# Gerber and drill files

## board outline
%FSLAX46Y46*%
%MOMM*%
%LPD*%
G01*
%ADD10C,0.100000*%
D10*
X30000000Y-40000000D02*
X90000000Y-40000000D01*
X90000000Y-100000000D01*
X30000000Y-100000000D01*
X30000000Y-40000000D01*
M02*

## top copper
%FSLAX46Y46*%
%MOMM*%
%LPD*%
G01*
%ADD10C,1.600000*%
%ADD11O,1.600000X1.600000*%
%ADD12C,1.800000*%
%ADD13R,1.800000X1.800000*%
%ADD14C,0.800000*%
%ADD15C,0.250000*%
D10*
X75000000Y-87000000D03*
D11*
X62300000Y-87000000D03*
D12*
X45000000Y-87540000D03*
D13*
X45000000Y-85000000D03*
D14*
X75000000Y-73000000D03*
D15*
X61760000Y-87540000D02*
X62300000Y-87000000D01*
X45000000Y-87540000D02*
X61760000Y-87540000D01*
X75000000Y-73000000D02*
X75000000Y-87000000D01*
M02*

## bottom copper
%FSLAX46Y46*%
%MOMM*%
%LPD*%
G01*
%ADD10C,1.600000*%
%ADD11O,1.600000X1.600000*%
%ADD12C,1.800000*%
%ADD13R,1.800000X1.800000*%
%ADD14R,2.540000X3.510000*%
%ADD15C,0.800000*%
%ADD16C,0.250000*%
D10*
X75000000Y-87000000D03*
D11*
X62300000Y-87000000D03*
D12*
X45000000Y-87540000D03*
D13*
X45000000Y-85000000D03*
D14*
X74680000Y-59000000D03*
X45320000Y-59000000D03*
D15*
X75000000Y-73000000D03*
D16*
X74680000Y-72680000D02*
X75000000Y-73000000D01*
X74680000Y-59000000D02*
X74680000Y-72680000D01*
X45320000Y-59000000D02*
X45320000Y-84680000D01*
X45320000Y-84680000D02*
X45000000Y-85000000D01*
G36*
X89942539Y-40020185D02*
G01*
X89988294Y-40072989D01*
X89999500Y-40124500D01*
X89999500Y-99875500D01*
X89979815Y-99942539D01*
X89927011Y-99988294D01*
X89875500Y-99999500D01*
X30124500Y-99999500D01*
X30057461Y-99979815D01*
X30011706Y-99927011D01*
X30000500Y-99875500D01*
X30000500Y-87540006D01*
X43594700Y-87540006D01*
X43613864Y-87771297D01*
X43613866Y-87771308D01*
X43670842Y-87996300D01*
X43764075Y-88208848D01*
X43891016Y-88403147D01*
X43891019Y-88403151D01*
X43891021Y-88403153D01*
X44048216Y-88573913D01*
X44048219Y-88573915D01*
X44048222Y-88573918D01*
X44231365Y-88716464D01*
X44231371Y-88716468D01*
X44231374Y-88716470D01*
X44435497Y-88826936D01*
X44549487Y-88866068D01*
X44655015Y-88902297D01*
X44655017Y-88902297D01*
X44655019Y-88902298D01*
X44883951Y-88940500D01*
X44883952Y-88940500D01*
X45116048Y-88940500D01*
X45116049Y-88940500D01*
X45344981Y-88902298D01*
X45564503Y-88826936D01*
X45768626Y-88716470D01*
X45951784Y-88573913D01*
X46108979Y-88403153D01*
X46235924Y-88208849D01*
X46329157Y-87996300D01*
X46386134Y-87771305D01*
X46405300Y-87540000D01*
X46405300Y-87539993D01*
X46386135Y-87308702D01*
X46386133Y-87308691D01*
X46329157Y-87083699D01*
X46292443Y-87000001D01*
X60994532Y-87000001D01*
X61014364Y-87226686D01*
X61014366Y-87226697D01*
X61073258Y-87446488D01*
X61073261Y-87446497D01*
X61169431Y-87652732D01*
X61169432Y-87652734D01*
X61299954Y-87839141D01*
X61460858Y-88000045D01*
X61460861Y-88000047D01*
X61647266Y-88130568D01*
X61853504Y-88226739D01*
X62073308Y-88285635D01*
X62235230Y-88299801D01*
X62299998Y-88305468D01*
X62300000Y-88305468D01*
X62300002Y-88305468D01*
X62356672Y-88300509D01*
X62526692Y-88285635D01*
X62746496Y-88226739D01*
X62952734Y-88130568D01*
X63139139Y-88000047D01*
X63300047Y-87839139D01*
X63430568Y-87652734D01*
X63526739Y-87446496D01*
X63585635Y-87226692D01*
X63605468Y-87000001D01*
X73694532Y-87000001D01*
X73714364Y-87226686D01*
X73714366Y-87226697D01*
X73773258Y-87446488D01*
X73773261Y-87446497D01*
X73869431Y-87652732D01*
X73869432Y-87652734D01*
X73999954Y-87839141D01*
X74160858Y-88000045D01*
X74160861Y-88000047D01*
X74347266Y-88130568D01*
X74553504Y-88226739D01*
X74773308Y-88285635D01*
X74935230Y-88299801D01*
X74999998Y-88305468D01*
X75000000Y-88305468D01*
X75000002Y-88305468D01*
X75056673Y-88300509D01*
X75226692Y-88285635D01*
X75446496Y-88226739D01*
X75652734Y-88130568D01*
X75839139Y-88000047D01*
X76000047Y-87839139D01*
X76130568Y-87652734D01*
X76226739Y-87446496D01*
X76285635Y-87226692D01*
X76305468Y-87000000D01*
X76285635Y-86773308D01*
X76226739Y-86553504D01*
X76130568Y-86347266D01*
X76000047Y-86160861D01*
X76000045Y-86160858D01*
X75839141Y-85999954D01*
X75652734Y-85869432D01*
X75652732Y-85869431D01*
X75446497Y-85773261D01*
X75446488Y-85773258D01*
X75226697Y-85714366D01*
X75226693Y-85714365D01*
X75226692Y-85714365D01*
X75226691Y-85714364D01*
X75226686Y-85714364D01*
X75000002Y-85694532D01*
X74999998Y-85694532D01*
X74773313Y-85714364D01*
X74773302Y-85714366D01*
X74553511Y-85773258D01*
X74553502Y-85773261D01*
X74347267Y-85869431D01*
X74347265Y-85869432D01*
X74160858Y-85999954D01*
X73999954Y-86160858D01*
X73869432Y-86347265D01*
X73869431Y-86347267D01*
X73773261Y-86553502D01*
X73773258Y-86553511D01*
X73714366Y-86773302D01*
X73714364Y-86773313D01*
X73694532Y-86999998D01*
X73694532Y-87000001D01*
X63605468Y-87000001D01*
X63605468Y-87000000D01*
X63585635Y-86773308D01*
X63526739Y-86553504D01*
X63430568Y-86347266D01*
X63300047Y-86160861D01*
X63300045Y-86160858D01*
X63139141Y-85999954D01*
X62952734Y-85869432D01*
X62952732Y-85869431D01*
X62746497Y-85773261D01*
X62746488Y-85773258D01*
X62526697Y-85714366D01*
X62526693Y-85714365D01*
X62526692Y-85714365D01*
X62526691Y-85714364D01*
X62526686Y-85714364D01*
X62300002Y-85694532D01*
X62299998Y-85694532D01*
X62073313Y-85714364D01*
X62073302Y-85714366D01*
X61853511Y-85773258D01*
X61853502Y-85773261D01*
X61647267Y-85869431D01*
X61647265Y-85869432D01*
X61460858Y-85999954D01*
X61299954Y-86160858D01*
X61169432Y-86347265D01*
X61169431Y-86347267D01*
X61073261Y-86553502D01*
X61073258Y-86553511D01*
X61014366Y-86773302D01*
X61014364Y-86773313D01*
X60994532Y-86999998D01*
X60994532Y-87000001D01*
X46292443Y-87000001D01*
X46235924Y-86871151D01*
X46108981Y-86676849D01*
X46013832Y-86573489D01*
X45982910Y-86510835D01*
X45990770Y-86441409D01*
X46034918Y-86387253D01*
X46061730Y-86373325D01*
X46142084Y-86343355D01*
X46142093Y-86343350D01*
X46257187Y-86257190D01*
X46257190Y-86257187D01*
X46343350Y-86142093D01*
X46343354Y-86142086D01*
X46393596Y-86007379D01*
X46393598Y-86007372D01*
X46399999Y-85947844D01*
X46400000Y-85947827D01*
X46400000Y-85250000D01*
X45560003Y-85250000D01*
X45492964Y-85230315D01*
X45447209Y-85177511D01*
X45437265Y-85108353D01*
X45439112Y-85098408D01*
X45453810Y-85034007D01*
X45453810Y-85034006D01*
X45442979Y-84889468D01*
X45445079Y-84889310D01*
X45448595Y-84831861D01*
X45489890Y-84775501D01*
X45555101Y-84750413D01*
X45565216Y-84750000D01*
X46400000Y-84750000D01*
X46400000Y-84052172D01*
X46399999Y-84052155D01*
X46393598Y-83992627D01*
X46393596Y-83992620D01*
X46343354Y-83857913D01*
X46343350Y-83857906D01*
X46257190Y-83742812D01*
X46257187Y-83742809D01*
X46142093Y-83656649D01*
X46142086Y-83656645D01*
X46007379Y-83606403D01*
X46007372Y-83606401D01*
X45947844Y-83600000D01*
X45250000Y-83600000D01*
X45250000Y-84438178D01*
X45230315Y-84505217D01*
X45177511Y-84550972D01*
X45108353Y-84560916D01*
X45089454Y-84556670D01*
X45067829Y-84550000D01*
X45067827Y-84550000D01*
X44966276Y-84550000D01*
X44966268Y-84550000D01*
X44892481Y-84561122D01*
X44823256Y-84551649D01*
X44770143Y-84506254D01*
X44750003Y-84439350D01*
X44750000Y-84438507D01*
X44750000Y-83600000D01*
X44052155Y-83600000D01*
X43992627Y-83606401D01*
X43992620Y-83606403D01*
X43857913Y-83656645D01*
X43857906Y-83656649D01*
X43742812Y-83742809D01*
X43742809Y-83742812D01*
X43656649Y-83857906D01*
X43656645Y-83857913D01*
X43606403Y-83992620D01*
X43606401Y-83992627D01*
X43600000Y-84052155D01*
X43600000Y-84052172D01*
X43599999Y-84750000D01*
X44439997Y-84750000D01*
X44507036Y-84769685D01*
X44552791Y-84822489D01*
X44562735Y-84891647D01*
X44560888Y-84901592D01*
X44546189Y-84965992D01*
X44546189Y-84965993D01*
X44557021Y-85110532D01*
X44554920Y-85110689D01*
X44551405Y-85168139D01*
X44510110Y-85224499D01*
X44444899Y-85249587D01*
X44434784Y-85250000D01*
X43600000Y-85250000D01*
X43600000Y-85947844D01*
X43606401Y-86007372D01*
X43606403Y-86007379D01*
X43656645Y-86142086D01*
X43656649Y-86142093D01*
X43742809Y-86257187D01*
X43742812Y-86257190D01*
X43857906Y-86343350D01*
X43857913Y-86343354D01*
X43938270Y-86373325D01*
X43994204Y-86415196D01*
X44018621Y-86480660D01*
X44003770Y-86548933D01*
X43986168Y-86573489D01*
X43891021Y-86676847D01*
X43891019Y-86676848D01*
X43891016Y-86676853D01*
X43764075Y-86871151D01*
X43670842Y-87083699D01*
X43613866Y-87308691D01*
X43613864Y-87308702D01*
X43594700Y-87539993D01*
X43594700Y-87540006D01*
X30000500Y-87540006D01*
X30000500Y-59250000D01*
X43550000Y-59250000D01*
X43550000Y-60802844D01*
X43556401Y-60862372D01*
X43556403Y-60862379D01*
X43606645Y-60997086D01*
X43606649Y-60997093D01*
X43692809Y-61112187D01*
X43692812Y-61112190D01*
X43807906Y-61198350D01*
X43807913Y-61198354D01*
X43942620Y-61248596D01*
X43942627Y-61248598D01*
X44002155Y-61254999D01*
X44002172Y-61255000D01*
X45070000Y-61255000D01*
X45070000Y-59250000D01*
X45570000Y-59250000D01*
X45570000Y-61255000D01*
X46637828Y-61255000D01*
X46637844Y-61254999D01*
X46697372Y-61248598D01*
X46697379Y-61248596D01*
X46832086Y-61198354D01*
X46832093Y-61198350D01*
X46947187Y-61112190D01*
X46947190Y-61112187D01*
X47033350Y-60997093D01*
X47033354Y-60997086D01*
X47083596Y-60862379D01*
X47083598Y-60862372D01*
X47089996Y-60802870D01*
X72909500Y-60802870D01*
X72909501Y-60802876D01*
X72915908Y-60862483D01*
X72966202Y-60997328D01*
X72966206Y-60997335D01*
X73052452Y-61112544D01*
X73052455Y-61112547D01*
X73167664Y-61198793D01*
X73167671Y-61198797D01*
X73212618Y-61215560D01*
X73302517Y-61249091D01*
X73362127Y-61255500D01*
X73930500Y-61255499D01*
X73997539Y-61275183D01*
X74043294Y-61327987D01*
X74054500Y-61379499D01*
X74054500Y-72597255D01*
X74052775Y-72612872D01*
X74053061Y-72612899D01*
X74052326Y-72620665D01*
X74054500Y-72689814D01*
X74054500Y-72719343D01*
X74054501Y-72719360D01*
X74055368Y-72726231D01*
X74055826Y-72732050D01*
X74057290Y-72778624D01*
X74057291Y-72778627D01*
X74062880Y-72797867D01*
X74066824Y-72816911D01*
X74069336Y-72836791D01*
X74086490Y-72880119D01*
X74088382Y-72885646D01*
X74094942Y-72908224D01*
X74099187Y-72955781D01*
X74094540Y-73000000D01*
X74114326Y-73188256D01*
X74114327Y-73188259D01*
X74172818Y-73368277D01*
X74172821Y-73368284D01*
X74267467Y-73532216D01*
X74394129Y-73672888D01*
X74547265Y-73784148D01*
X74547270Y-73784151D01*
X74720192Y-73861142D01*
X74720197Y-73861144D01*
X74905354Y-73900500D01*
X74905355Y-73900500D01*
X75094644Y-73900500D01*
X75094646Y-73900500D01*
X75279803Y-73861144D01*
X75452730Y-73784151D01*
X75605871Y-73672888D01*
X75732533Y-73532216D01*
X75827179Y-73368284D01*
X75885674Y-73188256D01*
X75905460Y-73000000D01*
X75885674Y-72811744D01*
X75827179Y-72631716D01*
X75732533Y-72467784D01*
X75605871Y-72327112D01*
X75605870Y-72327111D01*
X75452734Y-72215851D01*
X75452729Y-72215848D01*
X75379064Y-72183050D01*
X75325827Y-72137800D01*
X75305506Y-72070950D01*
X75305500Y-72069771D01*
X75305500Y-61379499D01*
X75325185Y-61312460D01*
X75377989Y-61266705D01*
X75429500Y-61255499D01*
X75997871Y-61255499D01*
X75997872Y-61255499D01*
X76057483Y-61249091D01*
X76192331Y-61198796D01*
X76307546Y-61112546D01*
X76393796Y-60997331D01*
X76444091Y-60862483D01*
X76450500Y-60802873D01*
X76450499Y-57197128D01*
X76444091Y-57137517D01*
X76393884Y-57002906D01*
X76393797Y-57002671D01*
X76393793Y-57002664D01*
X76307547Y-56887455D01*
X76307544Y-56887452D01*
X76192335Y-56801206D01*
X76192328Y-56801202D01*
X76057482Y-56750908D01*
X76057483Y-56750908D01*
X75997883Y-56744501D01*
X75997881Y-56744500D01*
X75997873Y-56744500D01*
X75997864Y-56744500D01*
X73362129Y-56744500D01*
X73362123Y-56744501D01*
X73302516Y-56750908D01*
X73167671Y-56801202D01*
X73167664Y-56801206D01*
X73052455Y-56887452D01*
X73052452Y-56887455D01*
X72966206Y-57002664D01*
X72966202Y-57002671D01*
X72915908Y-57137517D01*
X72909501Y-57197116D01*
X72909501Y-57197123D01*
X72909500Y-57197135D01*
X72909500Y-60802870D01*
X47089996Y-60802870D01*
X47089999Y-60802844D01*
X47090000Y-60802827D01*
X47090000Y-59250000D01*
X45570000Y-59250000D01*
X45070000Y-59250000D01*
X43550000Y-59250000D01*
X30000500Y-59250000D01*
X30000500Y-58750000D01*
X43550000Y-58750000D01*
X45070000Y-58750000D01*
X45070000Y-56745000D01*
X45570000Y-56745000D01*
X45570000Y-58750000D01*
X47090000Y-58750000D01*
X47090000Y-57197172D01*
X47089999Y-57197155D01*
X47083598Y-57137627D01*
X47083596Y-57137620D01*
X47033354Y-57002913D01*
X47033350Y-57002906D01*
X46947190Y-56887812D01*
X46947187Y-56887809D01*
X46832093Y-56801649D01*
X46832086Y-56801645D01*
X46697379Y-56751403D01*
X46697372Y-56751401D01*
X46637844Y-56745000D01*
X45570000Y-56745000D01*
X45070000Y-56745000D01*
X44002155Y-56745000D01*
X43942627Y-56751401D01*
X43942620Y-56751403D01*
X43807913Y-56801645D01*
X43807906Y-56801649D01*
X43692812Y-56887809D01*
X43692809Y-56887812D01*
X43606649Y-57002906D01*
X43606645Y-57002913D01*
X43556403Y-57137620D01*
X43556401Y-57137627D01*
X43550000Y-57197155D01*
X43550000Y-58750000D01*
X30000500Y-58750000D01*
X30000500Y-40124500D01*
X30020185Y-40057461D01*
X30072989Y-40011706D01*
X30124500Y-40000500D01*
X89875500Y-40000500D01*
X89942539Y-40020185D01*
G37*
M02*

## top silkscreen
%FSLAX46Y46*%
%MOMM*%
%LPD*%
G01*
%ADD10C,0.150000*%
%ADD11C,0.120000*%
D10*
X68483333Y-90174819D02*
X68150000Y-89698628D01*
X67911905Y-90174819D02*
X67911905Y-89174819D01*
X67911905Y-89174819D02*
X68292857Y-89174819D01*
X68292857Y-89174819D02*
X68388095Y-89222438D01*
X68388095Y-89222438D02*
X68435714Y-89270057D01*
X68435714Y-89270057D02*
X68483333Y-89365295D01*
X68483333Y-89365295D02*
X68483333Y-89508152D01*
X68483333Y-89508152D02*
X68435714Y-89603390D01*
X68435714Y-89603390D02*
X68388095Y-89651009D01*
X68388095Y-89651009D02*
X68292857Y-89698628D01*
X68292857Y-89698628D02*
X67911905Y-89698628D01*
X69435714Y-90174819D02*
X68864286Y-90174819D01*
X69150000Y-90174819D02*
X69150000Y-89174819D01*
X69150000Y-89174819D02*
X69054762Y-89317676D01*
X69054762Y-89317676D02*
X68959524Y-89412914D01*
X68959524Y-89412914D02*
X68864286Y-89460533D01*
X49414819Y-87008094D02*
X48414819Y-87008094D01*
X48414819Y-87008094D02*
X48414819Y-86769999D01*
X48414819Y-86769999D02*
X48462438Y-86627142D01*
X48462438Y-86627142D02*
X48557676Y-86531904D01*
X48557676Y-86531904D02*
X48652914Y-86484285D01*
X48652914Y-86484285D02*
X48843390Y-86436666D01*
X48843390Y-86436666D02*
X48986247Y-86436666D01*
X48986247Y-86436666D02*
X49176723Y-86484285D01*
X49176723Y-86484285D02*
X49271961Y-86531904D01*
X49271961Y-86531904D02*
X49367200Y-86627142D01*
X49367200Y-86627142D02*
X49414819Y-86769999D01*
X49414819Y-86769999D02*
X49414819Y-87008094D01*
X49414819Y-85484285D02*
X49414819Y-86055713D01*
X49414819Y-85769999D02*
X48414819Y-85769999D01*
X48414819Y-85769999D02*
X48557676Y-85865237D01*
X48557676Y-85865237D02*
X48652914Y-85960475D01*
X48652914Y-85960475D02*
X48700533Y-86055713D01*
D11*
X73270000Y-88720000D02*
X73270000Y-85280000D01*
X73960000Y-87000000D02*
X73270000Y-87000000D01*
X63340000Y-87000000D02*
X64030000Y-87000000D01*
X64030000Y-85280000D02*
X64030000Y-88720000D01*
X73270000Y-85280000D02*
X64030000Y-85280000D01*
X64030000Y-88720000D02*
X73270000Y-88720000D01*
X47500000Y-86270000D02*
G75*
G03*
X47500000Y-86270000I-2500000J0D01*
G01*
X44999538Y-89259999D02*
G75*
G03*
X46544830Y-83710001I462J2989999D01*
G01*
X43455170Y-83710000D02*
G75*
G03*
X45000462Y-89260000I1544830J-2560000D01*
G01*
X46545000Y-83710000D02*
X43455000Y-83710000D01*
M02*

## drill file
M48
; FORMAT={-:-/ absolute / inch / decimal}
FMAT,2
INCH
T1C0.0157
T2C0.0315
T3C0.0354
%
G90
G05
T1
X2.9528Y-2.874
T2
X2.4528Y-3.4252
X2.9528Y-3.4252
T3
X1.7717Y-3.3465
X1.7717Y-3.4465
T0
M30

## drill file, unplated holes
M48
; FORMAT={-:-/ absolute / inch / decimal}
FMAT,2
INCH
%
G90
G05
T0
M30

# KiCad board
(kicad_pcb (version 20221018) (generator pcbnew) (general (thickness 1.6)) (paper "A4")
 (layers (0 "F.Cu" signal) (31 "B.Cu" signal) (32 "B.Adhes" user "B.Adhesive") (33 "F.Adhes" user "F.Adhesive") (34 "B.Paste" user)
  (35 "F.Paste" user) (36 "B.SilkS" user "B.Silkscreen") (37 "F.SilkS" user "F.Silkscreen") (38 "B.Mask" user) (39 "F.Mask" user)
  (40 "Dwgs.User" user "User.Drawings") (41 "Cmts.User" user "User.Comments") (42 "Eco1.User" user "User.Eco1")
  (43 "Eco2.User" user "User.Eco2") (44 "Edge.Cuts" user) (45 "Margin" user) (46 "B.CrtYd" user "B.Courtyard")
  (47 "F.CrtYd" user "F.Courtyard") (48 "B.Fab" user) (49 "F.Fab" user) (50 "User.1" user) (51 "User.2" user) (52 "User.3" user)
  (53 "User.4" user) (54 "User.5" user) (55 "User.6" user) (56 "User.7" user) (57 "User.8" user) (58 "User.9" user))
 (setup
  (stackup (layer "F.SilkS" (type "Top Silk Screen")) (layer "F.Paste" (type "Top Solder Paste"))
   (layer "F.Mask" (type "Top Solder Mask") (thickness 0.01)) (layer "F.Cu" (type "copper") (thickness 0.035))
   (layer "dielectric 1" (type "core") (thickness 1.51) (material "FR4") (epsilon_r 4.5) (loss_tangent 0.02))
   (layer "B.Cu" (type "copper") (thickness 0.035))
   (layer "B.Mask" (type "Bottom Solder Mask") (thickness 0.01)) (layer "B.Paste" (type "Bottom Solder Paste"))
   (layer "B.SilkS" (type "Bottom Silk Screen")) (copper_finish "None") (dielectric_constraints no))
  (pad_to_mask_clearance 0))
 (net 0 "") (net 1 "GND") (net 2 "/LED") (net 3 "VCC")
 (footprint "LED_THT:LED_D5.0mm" (layer "F.Cu") (at 45 85 -90)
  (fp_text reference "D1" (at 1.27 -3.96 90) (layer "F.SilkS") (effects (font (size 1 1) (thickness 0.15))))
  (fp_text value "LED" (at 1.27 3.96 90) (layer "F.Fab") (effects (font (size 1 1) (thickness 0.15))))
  (fp_line (start -1.29 -1.545) (end -1.29 1.545) (stroke (width 0.12) (type solid)) (layer "F.SilkS"))
  (fp_arc (start -1.29 -1.54483) (mid 2.072002 -2.880433) (end 4.26 0.000462) (stroke (width 0.12) (type solid)) (layer "F.SilkS"))
  (fp_arc (start 4.26 -0.000462) (mid 2.072002 2.880433) (end -1.29 1.54483) (stroke (width 0.12) (type solid)) (layer "F.SilkS"))
  (fp_circle (center 1.27 0) (end 3.77 0) (stroke (width 0.12) (type solid)) (fill none) (layer "F.SilkS"))
  (pad "1" thru_hole rect (at 0 0 270) (size 1.8 1.8) (drill 0.9) (layers "*.Cu" "*.Mask") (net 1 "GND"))
  (pad "2" thru_hole circle (at 2.54 0 270) (size 1.8 1.8) (drill 0.9) (layers "*.Cu" "*.Mask") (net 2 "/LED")))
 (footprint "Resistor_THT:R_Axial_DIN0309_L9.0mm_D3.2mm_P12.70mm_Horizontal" (layer "F.Cu") (at 75 87 180)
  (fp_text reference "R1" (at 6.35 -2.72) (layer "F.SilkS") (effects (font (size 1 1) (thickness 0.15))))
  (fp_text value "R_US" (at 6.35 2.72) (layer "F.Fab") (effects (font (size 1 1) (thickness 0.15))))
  (fp_line (start 1.04 0) (end 1.73 0) (stroke (width 0.12) (type solid)) (layer "F.SilkS"))
  (fp_line (start 1.73 -1.72) (end 1.73 1.72) (stroke (width 0.12) (type solid)) (layer "F.SilkS"))
  (fp_line (start 1.73 1.72) (end 10.97 1.72) (stroke (width 0.12) (type solid)) (layer "F.SilkS"))
  (fp_line (start 10.97 -1.72) (end 1.73 -1.72) (stroke (width 0.12) (type solid)) (layer "F.SilkS"))
  (fp_line (start 10.97 1.72) (end 10.97 -1.72) (stroke (width 0.12) (type solid)) (layer "F.SilkS"))
  (fp_line (start 11.66 0) (end 10.97 0) (stroke (width 0.12) (type solid)) (layer "F.SilkS"))
  (pad "1" thru_hole circle (at 0 0 180) (size 1.6 1.6) (drill 0.8) (layers "*.Cu" "*.Mask") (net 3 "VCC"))
  (pad "2" thru_hole oval (at 12.7 0 180) (size 1.6 1.6) (drill 0.8) (layers "*.Cu" "*.Mask") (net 2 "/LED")))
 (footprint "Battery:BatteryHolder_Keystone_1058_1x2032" (layer "B.Cu") (at 60 59 180)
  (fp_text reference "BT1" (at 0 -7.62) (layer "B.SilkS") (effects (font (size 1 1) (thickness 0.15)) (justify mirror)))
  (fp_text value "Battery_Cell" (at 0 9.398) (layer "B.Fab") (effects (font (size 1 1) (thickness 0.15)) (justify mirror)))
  (pad "1" smd rect (at -14.68 0 180) (size 2.54 3.51) (layers "B.Cu" "B.Paste" "B.Mask") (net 3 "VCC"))
  (pad "2" smd rect (at 14.68 0 180) (size 2.54 3.51) (layers "B.Cu" "B.Paste" "B.Mask") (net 1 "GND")))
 (gr_rect (start 30 40) (end 90 100) (stroke (width 0.1) (type default)) (fill none) (layer "Edge.Cuts"))
 (segment (start 75 73) (end 75 87) (width 0.25) (layer "F.Cu") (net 3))
 (via (at 75 73) (size 0.8) (drill 0.4) (layers "F.Cu" "B.Cu") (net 3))
 (segment (start 74.68 59) (end 74.68 72.68) (width 0.25) (layer "B.Cu") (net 3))
 (segment (start 74.68 72.68) (end 75 73) (width 0.25) (layer "B.Cu") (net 3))
 (segment (start 45.32 59) (end 45.32 84.68) (width 0.25) (layer "B.Cu") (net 1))
 (segment (start 45.32 84.68) (end 45 85) (width 0.25) (layer "B.Cu") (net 1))
 (segment (start 61.76 87.54) (end 62.3 87) (width 0.25) (layer "F.Cu") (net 2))
 (segment (start 45 87.54) (end 61.76 87.54) (width 0.25) (layer "F.Cu") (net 2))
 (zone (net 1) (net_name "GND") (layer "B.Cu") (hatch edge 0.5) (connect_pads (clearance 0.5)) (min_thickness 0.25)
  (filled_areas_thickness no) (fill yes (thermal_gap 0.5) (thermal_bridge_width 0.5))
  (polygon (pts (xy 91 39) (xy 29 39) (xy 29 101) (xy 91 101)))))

